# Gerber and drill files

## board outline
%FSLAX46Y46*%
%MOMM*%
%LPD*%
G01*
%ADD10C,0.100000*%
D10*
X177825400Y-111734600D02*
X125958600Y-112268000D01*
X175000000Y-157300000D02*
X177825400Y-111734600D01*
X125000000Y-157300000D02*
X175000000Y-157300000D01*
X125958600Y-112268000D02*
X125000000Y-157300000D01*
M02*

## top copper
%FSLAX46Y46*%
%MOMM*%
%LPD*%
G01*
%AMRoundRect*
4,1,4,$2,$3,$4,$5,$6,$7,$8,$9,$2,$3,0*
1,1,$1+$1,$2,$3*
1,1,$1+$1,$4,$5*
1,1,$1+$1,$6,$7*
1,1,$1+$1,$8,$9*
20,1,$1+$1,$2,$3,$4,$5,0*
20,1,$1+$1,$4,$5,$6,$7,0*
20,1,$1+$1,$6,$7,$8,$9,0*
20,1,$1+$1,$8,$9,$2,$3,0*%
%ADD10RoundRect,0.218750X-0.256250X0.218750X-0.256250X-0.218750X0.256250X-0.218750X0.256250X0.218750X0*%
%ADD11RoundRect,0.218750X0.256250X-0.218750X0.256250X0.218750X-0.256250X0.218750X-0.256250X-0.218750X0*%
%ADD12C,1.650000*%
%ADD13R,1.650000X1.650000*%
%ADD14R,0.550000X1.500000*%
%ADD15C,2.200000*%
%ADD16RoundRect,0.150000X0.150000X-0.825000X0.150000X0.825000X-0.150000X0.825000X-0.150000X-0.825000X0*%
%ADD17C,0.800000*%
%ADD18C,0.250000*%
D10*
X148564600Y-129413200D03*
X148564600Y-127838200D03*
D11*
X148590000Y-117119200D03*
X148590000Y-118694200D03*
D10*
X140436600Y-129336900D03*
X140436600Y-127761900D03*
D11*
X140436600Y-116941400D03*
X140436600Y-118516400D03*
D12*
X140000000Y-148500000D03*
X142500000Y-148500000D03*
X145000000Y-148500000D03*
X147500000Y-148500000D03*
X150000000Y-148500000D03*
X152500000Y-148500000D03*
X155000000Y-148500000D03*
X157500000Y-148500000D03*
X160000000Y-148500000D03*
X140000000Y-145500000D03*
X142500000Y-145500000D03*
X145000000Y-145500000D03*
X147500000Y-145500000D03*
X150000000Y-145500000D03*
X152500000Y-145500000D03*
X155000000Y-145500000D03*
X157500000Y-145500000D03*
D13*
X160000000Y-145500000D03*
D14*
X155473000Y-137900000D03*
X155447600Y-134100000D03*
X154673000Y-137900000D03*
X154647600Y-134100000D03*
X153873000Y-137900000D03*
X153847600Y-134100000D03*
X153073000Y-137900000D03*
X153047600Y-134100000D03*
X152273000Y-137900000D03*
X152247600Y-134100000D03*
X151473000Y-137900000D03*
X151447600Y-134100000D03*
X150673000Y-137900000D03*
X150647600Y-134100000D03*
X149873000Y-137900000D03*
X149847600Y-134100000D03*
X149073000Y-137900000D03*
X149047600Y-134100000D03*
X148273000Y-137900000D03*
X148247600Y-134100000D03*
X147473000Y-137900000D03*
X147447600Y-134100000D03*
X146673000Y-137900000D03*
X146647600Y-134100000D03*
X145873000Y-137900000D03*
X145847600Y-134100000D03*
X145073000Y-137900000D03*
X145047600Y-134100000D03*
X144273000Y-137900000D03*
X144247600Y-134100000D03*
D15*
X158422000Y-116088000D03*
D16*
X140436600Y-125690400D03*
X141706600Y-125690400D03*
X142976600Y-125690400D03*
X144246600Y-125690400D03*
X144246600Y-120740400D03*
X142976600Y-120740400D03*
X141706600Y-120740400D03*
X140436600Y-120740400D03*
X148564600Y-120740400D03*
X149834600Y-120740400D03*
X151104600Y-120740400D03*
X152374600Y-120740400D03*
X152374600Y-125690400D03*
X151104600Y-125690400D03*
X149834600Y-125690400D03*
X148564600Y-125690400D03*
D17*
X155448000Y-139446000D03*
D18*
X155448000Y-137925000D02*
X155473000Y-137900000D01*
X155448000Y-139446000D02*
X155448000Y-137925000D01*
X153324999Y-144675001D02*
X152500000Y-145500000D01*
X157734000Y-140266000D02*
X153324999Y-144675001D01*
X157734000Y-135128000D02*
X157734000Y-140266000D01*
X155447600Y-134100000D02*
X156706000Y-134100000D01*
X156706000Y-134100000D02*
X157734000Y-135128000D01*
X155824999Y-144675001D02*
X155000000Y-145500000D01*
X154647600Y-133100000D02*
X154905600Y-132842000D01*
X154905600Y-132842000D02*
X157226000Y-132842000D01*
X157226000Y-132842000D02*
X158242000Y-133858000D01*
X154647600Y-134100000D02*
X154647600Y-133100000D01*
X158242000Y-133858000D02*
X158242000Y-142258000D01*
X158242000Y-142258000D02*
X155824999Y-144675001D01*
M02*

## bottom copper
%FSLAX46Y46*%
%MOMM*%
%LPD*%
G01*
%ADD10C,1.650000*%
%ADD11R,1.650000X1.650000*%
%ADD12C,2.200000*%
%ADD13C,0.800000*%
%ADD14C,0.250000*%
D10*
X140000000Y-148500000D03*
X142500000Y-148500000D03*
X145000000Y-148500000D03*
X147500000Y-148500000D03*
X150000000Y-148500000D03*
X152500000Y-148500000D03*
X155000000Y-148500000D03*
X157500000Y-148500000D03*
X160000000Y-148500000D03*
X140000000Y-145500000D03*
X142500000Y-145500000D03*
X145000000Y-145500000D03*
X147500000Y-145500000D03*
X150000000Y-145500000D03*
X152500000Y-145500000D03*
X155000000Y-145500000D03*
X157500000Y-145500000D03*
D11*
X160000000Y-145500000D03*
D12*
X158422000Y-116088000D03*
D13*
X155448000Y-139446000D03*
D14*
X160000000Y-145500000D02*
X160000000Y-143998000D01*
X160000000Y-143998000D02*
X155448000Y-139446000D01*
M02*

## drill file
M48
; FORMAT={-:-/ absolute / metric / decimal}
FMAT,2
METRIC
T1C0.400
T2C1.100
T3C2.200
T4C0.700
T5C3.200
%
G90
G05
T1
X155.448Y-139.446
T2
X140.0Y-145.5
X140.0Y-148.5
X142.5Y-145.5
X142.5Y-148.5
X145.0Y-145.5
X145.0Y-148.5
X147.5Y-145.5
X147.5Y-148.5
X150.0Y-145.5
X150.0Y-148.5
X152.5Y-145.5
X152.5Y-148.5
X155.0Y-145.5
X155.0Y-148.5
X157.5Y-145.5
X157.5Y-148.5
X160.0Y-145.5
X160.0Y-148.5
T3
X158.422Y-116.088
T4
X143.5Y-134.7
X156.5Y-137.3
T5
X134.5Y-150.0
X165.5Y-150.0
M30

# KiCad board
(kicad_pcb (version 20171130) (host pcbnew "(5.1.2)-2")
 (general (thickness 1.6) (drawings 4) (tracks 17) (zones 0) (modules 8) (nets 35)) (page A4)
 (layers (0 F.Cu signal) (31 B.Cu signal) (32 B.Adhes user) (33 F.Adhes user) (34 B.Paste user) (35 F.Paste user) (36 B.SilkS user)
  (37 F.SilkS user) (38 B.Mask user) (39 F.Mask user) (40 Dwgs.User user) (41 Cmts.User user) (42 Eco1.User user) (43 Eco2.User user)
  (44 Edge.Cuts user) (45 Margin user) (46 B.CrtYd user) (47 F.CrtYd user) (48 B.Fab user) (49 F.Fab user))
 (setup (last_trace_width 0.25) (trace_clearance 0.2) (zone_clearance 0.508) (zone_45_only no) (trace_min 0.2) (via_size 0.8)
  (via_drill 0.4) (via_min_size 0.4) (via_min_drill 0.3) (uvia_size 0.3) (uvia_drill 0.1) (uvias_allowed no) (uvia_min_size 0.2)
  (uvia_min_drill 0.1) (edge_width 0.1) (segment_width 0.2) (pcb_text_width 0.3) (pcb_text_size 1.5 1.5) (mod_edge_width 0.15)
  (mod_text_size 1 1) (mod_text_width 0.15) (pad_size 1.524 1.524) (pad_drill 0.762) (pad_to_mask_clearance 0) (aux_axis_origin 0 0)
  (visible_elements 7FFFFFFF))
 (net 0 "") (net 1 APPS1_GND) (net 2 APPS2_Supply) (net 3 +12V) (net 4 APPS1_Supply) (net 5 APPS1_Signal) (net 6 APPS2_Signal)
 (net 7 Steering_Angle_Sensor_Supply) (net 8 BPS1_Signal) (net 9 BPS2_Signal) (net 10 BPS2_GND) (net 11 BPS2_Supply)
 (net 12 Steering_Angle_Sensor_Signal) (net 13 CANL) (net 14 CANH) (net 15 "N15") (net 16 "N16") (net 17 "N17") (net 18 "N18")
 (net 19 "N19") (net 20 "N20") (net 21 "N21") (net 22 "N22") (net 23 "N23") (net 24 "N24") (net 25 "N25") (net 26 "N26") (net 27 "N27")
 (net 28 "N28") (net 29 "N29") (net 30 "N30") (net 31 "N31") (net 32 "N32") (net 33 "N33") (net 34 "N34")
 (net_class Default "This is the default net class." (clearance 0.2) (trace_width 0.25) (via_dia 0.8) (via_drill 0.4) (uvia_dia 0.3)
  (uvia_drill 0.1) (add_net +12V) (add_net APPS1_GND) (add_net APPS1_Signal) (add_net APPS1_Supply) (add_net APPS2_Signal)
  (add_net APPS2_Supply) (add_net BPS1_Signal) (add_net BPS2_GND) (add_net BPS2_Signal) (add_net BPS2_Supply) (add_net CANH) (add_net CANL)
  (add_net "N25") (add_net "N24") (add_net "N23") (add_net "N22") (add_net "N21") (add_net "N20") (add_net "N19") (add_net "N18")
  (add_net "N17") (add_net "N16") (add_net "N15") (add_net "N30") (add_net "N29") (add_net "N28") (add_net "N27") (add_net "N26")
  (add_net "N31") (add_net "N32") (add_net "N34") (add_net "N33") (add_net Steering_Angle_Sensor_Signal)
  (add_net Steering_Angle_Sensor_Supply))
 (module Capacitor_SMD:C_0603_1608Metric (layer F.Cu) (at 148.5646 128.6257 270)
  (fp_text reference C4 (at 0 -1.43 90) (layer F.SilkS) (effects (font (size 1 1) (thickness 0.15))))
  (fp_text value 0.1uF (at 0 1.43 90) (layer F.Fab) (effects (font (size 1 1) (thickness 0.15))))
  (pad 2 smd roundrect (at 0.7875 0 270) (size 0.875 0.95) (layers F.Cu F.Paste F.Mask) (roundrect_rratio 0.25) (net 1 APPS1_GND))
  (pad 1 smd roundrect (at -0.7875 0 270) (size 0.875 0.95) (layers F.Cu F.Paste F.Mask) (roundrect_rratio 0.25) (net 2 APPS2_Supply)))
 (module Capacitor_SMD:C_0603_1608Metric (layer F.Cu) (at 148.59 117.9067 90)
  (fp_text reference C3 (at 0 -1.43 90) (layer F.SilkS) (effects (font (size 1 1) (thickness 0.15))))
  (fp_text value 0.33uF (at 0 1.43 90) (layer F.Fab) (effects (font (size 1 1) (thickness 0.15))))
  (pad 2 smd roundrect (at 0.7875 0 90) (size 0.875 0.95) (layers F.Cu F.Paste F.Mask) (roundrect_rratio 0.25) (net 1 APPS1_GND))
  (pad 1 smd roundrect (at -0.7875 0 90) (size 0.875 0.95) (layers F.Cu F.Paste F.Mask) (roundrect_rratio 0.25) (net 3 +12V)))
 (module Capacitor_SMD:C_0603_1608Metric (layer F.Cu) (at 140.4366 128.5494 270)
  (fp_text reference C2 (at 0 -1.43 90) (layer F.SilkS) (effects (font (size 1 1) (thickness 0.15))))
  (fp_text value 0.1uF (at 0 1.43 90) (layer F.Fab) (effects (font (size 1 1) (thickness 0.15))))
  (pad 2 smd roundrect (at 0.7875 0 270) (size 0.875 0.95) (layers F.Cu F.Paste F.Mask) (roundrect_rratio 0.25) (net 1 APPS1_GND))
  (pad 1 smd roundrect (at -0.7875 0 270) (size 0.875 0.95) (layers F.Cu F.Paste F.Mask) (roundrect_rratio 0.25) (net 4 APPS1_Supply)))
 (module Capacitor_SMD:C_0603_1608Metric (layer F.Cu) (at 140.4366 117.7289 90)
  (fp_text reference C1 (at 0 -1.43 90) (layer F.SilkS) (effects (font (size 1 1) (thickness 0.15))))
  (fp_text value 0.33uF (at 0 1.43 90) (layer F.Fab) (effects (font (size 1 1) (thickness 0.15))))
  (pad 2 smd roundrect (at 0.7875 0 90) (size 0.875 0.95) (layers F.Cu F.Paste F.Mask) (roundrect_rratio 0.25) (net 1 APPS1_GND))
  (pad 1 smd roundrect (at -0.7875 0 90) (size 0.875 0.95) (layers F.Cu F.Paste F.Mask) (roundrect_rratio 0.25) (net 3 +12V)))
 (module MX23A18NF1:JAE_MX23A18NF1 (layer F.Cu) (at 150 150)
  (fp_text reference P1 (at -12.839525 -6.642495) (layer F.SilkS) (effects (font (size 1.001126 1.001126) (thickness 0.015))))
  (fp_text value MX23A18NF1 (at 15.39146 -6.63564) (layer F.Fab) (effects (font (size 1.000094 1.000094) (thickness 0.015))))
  (pad 18 thru_hole circle (at -10 -1.5) (size 1.65 1.65) (drill 1.1) (layers *.Cu *.Mask) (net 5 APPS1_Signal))
  (pad 17 thru_hole circle (at -7.5 -1.5) (size 1.65 1.65) (drill 1.1) (layers *.Cu *.Mask) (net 1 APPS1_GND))
  (pad 16 thru_hole circle (at -5 -1.5) (size 1.65 1.65) (drill 1.1) (layers *.Cu *.Mask) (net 4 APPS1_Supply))
  (pad 15 thru_hole circle (at -2.5 -1.5) (size 1.65 1.65) (drill 1.1) (layers *.Cu *.Mask) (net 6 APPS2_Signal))
  (pad 14 thru_hole circle (at 0 -1.5) (size 1.65 1.65) (drill 1.1) (layers *.Cu *.Mask) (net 1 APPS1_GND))
  (pad 13 thru_hole circle (at 2.5 -1.5) (size 1.65 1.65) (drill 1.1) (layers *.Cu *.Mask) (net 2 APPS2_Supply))
  (pad "" np_thru_hole circle (at 15.5 0) (size 3.2 3.2) (drill 3.2) (layers *.Cu *.Mask))
  (pad "" np_thru_hole circle (at -15.5 0) (size 3.2 3.2) (drill 3.2) (layers *.Cu *.Mask))
  (pad 12 thru_hole circle (at 5 -1.5) (size 1.65 1.65) (drill 1.1) (layers *.Cu *.Mask) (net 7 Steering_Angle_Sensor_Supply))
  (pad 11 thru_hole circle (at 7.5 -1.5) (size 1.65 1.65) (drill 1.1) (layers *.Cu *.Mask) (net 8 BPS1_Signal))
  (pad 10 thru_hole circle (at 10 -1.5) (size 1.65 1.65) (drill 1.1) (layers *.Cu *.Mask) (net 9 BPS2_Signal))
  (pad 9 thru_hole circle (at -10 -4.5) (size 1.65 1.65) (drill 1.1) (layers *.Cu *.Mask) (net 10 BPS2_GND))
  (pad 8 thru_hole circle (at -7.5 -4.5) (size 1.65 1.65) (drill 1.1) (layers *.Cu *.Mask) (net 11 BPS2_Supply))
  (pad 7 thru_hole circle (at -5 -4.5 90) (size 1.65 1.65) (drill 1.1) (layers *.Cu *.Mask) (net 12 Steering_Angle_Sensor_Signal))
  (pad 6 thru_hole circle (at -2.5 -4.5) (size 1.65 1.65) (drill 1.1) (layers *.Cu *.Mask) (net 1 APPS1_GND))
  (pad 5 thru_hole circle (at 0 -4.5) (size 1.65 1.65) (drill 1.1) (layers *.Cu *.Mask) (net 7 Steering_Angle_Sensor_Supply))
  (pad 4 thru_hole circle (at 2.5 -4.5) (size 1.65 1.65) (drill 1.1) (layers *.Cu *.Mask) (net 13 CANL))
  (pad 3 thru_hole circle (at 5 -4.5) (size 1.65 1.65) (drill 1.1) (layers *.Cu *.Mask) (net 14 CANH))
  (pad 2 thru_hole circle (at 7.5 -4.5) (size 1.65 1.65) (drill 1.1) (layers *.Cu *.Mask) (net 1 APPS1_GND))
  (pad 1 thru_hole rect (at 10 -4.5) (size 1.65 1.65) (drill 1.1) (layers *.Cu *.Mask) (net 3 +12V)))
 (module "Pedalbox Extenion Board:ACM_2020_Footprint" (layer F.Cu) (at 150 136 180)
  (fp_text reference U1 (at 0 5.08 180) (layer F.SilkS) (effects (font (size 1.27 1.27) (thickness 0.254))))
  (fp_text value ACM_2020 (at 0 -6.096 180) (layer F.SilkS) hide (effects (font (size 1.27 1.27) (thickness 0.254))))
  (pad 30 smd rect (at -5.473 -1.9 180) (size 0.55 1.5) (layers F.Cu F.Paste F.Mask) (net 3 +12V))
  (pad 29 smd rect (at -5.4476 1.9 180) (size 0.55 1.5) (layers F.Cu F.Paste F.Mask) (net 13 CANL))
  (pad 28 smd rect (at -4.673 -1.9 180) (size 0.55 1.5) (layers F.Cu F.Paste F.Mask) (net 7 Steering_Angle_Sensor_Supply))
  (pad 27 smd rect (at -4.6476 1.9 180) (size 0.55 1.5) (layers F.Cu F.Paste F.Mask) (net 14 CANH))
  (pad 26 smd rect (at -3.873 -1.9 180) (size 0.55 1.5) (layers F.Cu F.Paste F.Mask) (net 7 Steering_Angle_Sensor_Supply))
  (pad 25 smd rect (at -3.8476 1.9 180) (size 0.55 1.5) (layers F.Cu F.Paste F.Mask) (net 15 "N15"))
  (pad 24 smd rect (at -3.073 -1.9 180) (size 0.55 1.5) (layers F.Cu F.Paste F.Mask) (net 7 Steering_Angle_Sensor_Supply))
  (pad 23 smd rect (at -3.0476 1.9 180) (size 0.55 1.5) (layers F.Cu F.Paste F.Mask) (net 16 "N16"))
  (pad 22 smd rect (at -2.273 -1.9 180) (size 0.55 1.5) (layers F.Cu F.Paste F.Mask) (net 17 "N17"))
  (pad 21 smd rect (at -2.2476 1.9 180) (size 0.55 1.5) (layers F.Cu F.Paste F.Mask) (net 1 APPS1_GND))
  (pad 20 smd rect (at -1.473 -1.9 180) (size 0.55 1.5) (layers F.Cu F.Paste F.Mask) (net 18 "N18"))
  (pad 19 smd rect (at -1.4476 1.9 180) (size 0.55 1.5) (layers F.Cu F.Paste F.Mask) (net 1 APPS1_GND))
  (pad 18 smd rect (at -0.673 -1.9 180) (size 0.55 1.5) (layers F.Cu F.Paste F.Mask) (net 1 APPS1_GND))
  (pad 17 smd rect (at -0.6476 1.9 180) (size 0.55 1.5) (layers F.Cu F.Paste F.Mask) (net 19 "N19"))
  (pad 16 smd rect (at 0.127 -1.9 180) (size 0.55 1.5) (layers F.Cu F.Paste F.Mask) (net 1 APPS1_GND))
  (pad 15 smd rect (at 0.1524 1.9 180) (size 0.55 1.5) (layers F.Cu F.Paste F.Mask) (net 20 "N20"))
  (pad 14 smd rect (at 0.927 -1.9 180) (size 0.55 1.5) (layers F.Cu F.Paste F.Mask) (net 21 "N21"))
  (pad 13 smd rect (at 0.9524 1.9 180) (size 0.55 1.5) (layers F.Cu F.Paste F.Mask) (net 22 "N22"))
  (pad 12 smd rect (at 1.727 -1.9 180) (size 0.55 1.5) (layers F.Cu F.Paste F.Mask) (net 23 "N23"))
  (pad 11 smd rect (at 1.7524 1.9 180) (size 0.55 1.5) (layers F.Cu F.Paste F.Mask) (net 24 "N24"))
  (pad 10 smd rect (at 2.527 -1.9 180) (size 0.55 1.5) (layers F.Cu F.Paste F.Mask) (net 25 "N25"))
  (pad 9 smd rect (at 2.5524 1.9 180) (size 0.55 1.5) (layers F.Cu F.Paste F.Mask) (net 1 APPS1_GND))
  (pad 8 smd rect (at 3.327 -1.9 180) (size 0.55 1.5) (layers F.Cu F.Paste F.Mask) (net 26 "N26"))
  (pad 7 smd rect (at 3.3524 1.9 180) (size 0.55 1.5) (layers F.Cu F.Paste F.Mask) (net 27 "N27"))
  (pad 6 smd rect (at 4.127 -1.9 180) (size 0.55 1.5) (layers F.Cu F.Paste F.Mask) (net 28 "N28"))
  (pad 5 smd rect (at 4.1524 1.9 180) (size 0.55 1.5) (layers F.Cu F.Paste F.Mask) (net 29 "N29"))
  (pad 4 smd rect (at 4.927 -1.9 180) (size 0.55 1.5) (layers F.Cu F.Paste F.Mask) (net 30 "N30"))
  (pad 3 smd rect (at 4.9524 1.9 180) (size 0.55 1.5) (layers F.Cu F.Paste F.Mask) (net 5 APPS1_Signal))
  (pad 2 smd rect (at 5.727 -1.9 180) (size 0.55 1.5) (layers F.Cu F.Paste F.Mask) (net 6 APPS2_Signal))
  (pad 1 smd rect (at 5.7524 1.9 180) (size 0.55 1.5) (layers F.Cu F.Paste F.Mask) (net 12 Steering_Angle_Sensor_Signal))
  (pad "" np_thru_hole circle (at -6.5 -1.3 180) (size 0.7 0.7) (drill 0.7) (layers *.Cu *.Mask))
  (pad "" np_thru_hole circle (at 6.5 1.3 180) (size 0.7 0.7) (drill 0.7) (layers *.Cu *.Mask))
  (pad "" thru_hole circle (at -8.422 19.912 180) (size 2.2 2.2) (drill 2.2) (layers *.Cu *.Mask)))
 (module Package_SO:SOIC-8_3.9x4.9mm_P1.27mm (layer F.Cu) (at 142.3416 123.2154 90)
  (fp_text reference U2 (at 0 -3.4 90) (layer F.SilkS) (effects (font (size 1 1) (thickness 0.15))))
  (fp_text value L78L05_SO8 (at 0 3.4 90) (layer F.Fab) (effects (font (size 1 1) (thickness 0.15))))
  (pad 1 smd roundrect (at -2.475 -1.905 90) (size 1.95 0.6) (layers F.Cu F.Paste F.Mask) (roundrect_rratio 0.25) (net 4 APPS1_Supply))
  (pad 2 smd roundrect (at -2.475 -0.635 90) (size 1.95 0.6) (layers F.Cu F.Paste F.Mask) (roundrect_rratio 0.25) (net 1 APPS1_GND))
  (pad 3 smd roundrect (at -2.475 0.635 90) (size 1.95 0.6) (layers F.Cu F.Paste F.Mask) (roundrect_rratio 0.25) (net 1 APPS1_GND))
  (pad 4 smd roundrect (at -2.475 1.905 90) (size 1.95 0.6) (layers F.Cu F.Paste F.Mask) (roundrect_rratio 0.25) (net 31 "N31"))
  (pad 5 smd roundrect (at 2.475 1.905 90) (size 1.95 0.6) (layers F.Cu F.Paste F.Mask) (roundrect_rratio 0.25) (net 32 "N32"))
  (pad 6 smd roundrect (at 2.475 0.635 90) (size 1.95 0.6) (layers F.Cu F.Paste F.Mask) (roundrect_rratio 0.25) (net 1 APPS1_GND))
  (pad 7 smd roundrect (at 2.475 -0.635 90) (size 1.95 0.6) (layers F.Cu F.Paste F.Mask) (roundrect_rratio 0.25) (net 1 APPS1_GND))
  (pad 8 smd roundrect (at 2.475 -1.905 90) (size 1.95 0.6) (layers F.Cu F.Paste F.Mask) (roundrect_rratio 0.25) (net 3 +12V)))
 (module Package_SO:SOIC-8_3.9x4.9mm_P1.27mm (layer F.Cu) (at 150.4696 123.2154 90)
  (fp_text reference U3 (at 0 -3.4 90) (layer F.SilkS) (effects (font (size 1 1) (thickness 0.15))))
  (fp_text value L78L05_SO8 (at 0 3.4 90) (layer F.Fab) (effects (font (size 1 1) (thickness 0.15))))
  (pad 8 smd roundrect (at 2.475 -1.905 90) (size 1.95 0.6) (layers F.Cu F.Paste F.Mask) (roundrect_rratio 0.25) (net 3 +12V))
  (pad 7 smd roundrect (at 2.475 -0.635 90) (size 1.95 0.6) (layers F.Cu F.Paste F.Mask) (roundrect_rratio 0.25) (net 1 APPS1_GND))
  (pad 6 smd roundrect (at 2.475 0.635 90) (size 1.95 0.6) (layers F.Cu F.Paste F.Mask) (roundrect_rratio 0.25) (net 1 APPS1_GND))
  (pad 5 smd roundrect (at 2.475 1.905 90) (size 1.95 0.6) (layers F.Cu F.Paste F.Mask) (roundrect_rratio 0.25) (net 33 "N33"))
  (pad 4 smd roundrect (at -2.475 1.905 90) (size 1.95 0.6) (layers F.Cu F.Paste F.Mask) (roundrect_rratio 0.25) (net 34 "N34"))
  (pad 3 smd roundrect (at -2.475 0.635 90) (size 1.95 0.6) (layers F.Cu F.Paste F.Mask) (roundrect_rratio 0.25) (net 1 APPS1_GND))
  (pad 2 smd roundrect (at -2.475 -0.635 90) (size 1.95 0.6) (layers F.Cu F.Paste F.Mask) (roundrect_rratio 0.25) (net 1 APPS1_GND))
  (pad 1 smd roundrect (at -2.475 -1.905 90) (size 1.95 0.6) (layers F.Cu F.Paste F.Mask) (roundrect_rratio 0.25) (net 2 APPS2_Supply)))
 (gr_line (start 177.8254 111.7346) (end 125.9586 112.268) (layer Edge.Cuts) (width 0.1))
 (gr_line (start 175 157.3) (end 177.8254 111.7346) (layer Edge.Cuts) (width 0.1))
 (gr_line (start 125 157.3) (end 175 157.3) (layer Edge.Cuts) (width 0.1))
 (gr_line (start 125.9586 112.268) (end 125 157.3) (layer Edge.Cuts) (width 0.1))
 (via (at 155.448 139.446) (size 0.8) (drill 0.4) (layers F.Cu B.Cu) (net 3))
 (segment (start 160 145.5) (end 160 143.998) (width 0.25) (layer B.Cu) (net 3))
 (segment (start 160 143.998) (end 155.448 139.446) (width 0.25) (layer B.Cu) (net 3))
 (segment (start 155.448 137.925) (end 155.473 137.9) (width 0.25) (layer F.Cu) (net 3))
 (segment (start 155.448 139.446) (end 155.448 137.925) (width 0.25) (layer F.Cu) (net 3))
 (segment (start 153.324999 144.675001) (end 152.5 145.5) (width 0.25) (layer F.Cu) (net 13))
 (segment (start 157.734 140.266) (end 153.324999 144.675001) (width 0.25) (layer F.Cu) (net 13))
 (segment (start 157.734 135.128) (end 157.734 140.266) (width 0.25) (layer F.Cu) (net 13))
 (segment (start 155.4476 134.1) (end 156.706 134.1) (width 0.25) (layer F.Cu) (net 13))
 (segment (start 156.706 134.1) (end 157.734 135.128) (width 0.25) (layer F.Cu) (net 13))
 (segment (start 155.824999 144.675001) (end 155 145.5) (width 0.25) (layer F.Cu) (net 14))
 (segment (start 154.6476 133.1) (end 154.9056 132.842) (width 0.25) (layer F.Cu) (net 14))
 (segment (start 154.9056 132.842) (end 157.226 132.842) (width 0.25) (layer F.Cu) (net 14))
 (segment (start 157.226 132.842) (end 158.242 133.858) (width 0.25) (layer F.Cu) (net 14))
 (segment (start 154.6476 134.1) (end 154.6476 133.1) (width 0.25) (layer F.Cu) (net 14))
 (segment (start 158.242 133.858) (end 158.242 142.258) (width 0.25) (layer F.Cu) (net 14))
 (segment (start 158.242 142.258) (end 155.824999 144.675001) (width 0.25) (layer F.Cu) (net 14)))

